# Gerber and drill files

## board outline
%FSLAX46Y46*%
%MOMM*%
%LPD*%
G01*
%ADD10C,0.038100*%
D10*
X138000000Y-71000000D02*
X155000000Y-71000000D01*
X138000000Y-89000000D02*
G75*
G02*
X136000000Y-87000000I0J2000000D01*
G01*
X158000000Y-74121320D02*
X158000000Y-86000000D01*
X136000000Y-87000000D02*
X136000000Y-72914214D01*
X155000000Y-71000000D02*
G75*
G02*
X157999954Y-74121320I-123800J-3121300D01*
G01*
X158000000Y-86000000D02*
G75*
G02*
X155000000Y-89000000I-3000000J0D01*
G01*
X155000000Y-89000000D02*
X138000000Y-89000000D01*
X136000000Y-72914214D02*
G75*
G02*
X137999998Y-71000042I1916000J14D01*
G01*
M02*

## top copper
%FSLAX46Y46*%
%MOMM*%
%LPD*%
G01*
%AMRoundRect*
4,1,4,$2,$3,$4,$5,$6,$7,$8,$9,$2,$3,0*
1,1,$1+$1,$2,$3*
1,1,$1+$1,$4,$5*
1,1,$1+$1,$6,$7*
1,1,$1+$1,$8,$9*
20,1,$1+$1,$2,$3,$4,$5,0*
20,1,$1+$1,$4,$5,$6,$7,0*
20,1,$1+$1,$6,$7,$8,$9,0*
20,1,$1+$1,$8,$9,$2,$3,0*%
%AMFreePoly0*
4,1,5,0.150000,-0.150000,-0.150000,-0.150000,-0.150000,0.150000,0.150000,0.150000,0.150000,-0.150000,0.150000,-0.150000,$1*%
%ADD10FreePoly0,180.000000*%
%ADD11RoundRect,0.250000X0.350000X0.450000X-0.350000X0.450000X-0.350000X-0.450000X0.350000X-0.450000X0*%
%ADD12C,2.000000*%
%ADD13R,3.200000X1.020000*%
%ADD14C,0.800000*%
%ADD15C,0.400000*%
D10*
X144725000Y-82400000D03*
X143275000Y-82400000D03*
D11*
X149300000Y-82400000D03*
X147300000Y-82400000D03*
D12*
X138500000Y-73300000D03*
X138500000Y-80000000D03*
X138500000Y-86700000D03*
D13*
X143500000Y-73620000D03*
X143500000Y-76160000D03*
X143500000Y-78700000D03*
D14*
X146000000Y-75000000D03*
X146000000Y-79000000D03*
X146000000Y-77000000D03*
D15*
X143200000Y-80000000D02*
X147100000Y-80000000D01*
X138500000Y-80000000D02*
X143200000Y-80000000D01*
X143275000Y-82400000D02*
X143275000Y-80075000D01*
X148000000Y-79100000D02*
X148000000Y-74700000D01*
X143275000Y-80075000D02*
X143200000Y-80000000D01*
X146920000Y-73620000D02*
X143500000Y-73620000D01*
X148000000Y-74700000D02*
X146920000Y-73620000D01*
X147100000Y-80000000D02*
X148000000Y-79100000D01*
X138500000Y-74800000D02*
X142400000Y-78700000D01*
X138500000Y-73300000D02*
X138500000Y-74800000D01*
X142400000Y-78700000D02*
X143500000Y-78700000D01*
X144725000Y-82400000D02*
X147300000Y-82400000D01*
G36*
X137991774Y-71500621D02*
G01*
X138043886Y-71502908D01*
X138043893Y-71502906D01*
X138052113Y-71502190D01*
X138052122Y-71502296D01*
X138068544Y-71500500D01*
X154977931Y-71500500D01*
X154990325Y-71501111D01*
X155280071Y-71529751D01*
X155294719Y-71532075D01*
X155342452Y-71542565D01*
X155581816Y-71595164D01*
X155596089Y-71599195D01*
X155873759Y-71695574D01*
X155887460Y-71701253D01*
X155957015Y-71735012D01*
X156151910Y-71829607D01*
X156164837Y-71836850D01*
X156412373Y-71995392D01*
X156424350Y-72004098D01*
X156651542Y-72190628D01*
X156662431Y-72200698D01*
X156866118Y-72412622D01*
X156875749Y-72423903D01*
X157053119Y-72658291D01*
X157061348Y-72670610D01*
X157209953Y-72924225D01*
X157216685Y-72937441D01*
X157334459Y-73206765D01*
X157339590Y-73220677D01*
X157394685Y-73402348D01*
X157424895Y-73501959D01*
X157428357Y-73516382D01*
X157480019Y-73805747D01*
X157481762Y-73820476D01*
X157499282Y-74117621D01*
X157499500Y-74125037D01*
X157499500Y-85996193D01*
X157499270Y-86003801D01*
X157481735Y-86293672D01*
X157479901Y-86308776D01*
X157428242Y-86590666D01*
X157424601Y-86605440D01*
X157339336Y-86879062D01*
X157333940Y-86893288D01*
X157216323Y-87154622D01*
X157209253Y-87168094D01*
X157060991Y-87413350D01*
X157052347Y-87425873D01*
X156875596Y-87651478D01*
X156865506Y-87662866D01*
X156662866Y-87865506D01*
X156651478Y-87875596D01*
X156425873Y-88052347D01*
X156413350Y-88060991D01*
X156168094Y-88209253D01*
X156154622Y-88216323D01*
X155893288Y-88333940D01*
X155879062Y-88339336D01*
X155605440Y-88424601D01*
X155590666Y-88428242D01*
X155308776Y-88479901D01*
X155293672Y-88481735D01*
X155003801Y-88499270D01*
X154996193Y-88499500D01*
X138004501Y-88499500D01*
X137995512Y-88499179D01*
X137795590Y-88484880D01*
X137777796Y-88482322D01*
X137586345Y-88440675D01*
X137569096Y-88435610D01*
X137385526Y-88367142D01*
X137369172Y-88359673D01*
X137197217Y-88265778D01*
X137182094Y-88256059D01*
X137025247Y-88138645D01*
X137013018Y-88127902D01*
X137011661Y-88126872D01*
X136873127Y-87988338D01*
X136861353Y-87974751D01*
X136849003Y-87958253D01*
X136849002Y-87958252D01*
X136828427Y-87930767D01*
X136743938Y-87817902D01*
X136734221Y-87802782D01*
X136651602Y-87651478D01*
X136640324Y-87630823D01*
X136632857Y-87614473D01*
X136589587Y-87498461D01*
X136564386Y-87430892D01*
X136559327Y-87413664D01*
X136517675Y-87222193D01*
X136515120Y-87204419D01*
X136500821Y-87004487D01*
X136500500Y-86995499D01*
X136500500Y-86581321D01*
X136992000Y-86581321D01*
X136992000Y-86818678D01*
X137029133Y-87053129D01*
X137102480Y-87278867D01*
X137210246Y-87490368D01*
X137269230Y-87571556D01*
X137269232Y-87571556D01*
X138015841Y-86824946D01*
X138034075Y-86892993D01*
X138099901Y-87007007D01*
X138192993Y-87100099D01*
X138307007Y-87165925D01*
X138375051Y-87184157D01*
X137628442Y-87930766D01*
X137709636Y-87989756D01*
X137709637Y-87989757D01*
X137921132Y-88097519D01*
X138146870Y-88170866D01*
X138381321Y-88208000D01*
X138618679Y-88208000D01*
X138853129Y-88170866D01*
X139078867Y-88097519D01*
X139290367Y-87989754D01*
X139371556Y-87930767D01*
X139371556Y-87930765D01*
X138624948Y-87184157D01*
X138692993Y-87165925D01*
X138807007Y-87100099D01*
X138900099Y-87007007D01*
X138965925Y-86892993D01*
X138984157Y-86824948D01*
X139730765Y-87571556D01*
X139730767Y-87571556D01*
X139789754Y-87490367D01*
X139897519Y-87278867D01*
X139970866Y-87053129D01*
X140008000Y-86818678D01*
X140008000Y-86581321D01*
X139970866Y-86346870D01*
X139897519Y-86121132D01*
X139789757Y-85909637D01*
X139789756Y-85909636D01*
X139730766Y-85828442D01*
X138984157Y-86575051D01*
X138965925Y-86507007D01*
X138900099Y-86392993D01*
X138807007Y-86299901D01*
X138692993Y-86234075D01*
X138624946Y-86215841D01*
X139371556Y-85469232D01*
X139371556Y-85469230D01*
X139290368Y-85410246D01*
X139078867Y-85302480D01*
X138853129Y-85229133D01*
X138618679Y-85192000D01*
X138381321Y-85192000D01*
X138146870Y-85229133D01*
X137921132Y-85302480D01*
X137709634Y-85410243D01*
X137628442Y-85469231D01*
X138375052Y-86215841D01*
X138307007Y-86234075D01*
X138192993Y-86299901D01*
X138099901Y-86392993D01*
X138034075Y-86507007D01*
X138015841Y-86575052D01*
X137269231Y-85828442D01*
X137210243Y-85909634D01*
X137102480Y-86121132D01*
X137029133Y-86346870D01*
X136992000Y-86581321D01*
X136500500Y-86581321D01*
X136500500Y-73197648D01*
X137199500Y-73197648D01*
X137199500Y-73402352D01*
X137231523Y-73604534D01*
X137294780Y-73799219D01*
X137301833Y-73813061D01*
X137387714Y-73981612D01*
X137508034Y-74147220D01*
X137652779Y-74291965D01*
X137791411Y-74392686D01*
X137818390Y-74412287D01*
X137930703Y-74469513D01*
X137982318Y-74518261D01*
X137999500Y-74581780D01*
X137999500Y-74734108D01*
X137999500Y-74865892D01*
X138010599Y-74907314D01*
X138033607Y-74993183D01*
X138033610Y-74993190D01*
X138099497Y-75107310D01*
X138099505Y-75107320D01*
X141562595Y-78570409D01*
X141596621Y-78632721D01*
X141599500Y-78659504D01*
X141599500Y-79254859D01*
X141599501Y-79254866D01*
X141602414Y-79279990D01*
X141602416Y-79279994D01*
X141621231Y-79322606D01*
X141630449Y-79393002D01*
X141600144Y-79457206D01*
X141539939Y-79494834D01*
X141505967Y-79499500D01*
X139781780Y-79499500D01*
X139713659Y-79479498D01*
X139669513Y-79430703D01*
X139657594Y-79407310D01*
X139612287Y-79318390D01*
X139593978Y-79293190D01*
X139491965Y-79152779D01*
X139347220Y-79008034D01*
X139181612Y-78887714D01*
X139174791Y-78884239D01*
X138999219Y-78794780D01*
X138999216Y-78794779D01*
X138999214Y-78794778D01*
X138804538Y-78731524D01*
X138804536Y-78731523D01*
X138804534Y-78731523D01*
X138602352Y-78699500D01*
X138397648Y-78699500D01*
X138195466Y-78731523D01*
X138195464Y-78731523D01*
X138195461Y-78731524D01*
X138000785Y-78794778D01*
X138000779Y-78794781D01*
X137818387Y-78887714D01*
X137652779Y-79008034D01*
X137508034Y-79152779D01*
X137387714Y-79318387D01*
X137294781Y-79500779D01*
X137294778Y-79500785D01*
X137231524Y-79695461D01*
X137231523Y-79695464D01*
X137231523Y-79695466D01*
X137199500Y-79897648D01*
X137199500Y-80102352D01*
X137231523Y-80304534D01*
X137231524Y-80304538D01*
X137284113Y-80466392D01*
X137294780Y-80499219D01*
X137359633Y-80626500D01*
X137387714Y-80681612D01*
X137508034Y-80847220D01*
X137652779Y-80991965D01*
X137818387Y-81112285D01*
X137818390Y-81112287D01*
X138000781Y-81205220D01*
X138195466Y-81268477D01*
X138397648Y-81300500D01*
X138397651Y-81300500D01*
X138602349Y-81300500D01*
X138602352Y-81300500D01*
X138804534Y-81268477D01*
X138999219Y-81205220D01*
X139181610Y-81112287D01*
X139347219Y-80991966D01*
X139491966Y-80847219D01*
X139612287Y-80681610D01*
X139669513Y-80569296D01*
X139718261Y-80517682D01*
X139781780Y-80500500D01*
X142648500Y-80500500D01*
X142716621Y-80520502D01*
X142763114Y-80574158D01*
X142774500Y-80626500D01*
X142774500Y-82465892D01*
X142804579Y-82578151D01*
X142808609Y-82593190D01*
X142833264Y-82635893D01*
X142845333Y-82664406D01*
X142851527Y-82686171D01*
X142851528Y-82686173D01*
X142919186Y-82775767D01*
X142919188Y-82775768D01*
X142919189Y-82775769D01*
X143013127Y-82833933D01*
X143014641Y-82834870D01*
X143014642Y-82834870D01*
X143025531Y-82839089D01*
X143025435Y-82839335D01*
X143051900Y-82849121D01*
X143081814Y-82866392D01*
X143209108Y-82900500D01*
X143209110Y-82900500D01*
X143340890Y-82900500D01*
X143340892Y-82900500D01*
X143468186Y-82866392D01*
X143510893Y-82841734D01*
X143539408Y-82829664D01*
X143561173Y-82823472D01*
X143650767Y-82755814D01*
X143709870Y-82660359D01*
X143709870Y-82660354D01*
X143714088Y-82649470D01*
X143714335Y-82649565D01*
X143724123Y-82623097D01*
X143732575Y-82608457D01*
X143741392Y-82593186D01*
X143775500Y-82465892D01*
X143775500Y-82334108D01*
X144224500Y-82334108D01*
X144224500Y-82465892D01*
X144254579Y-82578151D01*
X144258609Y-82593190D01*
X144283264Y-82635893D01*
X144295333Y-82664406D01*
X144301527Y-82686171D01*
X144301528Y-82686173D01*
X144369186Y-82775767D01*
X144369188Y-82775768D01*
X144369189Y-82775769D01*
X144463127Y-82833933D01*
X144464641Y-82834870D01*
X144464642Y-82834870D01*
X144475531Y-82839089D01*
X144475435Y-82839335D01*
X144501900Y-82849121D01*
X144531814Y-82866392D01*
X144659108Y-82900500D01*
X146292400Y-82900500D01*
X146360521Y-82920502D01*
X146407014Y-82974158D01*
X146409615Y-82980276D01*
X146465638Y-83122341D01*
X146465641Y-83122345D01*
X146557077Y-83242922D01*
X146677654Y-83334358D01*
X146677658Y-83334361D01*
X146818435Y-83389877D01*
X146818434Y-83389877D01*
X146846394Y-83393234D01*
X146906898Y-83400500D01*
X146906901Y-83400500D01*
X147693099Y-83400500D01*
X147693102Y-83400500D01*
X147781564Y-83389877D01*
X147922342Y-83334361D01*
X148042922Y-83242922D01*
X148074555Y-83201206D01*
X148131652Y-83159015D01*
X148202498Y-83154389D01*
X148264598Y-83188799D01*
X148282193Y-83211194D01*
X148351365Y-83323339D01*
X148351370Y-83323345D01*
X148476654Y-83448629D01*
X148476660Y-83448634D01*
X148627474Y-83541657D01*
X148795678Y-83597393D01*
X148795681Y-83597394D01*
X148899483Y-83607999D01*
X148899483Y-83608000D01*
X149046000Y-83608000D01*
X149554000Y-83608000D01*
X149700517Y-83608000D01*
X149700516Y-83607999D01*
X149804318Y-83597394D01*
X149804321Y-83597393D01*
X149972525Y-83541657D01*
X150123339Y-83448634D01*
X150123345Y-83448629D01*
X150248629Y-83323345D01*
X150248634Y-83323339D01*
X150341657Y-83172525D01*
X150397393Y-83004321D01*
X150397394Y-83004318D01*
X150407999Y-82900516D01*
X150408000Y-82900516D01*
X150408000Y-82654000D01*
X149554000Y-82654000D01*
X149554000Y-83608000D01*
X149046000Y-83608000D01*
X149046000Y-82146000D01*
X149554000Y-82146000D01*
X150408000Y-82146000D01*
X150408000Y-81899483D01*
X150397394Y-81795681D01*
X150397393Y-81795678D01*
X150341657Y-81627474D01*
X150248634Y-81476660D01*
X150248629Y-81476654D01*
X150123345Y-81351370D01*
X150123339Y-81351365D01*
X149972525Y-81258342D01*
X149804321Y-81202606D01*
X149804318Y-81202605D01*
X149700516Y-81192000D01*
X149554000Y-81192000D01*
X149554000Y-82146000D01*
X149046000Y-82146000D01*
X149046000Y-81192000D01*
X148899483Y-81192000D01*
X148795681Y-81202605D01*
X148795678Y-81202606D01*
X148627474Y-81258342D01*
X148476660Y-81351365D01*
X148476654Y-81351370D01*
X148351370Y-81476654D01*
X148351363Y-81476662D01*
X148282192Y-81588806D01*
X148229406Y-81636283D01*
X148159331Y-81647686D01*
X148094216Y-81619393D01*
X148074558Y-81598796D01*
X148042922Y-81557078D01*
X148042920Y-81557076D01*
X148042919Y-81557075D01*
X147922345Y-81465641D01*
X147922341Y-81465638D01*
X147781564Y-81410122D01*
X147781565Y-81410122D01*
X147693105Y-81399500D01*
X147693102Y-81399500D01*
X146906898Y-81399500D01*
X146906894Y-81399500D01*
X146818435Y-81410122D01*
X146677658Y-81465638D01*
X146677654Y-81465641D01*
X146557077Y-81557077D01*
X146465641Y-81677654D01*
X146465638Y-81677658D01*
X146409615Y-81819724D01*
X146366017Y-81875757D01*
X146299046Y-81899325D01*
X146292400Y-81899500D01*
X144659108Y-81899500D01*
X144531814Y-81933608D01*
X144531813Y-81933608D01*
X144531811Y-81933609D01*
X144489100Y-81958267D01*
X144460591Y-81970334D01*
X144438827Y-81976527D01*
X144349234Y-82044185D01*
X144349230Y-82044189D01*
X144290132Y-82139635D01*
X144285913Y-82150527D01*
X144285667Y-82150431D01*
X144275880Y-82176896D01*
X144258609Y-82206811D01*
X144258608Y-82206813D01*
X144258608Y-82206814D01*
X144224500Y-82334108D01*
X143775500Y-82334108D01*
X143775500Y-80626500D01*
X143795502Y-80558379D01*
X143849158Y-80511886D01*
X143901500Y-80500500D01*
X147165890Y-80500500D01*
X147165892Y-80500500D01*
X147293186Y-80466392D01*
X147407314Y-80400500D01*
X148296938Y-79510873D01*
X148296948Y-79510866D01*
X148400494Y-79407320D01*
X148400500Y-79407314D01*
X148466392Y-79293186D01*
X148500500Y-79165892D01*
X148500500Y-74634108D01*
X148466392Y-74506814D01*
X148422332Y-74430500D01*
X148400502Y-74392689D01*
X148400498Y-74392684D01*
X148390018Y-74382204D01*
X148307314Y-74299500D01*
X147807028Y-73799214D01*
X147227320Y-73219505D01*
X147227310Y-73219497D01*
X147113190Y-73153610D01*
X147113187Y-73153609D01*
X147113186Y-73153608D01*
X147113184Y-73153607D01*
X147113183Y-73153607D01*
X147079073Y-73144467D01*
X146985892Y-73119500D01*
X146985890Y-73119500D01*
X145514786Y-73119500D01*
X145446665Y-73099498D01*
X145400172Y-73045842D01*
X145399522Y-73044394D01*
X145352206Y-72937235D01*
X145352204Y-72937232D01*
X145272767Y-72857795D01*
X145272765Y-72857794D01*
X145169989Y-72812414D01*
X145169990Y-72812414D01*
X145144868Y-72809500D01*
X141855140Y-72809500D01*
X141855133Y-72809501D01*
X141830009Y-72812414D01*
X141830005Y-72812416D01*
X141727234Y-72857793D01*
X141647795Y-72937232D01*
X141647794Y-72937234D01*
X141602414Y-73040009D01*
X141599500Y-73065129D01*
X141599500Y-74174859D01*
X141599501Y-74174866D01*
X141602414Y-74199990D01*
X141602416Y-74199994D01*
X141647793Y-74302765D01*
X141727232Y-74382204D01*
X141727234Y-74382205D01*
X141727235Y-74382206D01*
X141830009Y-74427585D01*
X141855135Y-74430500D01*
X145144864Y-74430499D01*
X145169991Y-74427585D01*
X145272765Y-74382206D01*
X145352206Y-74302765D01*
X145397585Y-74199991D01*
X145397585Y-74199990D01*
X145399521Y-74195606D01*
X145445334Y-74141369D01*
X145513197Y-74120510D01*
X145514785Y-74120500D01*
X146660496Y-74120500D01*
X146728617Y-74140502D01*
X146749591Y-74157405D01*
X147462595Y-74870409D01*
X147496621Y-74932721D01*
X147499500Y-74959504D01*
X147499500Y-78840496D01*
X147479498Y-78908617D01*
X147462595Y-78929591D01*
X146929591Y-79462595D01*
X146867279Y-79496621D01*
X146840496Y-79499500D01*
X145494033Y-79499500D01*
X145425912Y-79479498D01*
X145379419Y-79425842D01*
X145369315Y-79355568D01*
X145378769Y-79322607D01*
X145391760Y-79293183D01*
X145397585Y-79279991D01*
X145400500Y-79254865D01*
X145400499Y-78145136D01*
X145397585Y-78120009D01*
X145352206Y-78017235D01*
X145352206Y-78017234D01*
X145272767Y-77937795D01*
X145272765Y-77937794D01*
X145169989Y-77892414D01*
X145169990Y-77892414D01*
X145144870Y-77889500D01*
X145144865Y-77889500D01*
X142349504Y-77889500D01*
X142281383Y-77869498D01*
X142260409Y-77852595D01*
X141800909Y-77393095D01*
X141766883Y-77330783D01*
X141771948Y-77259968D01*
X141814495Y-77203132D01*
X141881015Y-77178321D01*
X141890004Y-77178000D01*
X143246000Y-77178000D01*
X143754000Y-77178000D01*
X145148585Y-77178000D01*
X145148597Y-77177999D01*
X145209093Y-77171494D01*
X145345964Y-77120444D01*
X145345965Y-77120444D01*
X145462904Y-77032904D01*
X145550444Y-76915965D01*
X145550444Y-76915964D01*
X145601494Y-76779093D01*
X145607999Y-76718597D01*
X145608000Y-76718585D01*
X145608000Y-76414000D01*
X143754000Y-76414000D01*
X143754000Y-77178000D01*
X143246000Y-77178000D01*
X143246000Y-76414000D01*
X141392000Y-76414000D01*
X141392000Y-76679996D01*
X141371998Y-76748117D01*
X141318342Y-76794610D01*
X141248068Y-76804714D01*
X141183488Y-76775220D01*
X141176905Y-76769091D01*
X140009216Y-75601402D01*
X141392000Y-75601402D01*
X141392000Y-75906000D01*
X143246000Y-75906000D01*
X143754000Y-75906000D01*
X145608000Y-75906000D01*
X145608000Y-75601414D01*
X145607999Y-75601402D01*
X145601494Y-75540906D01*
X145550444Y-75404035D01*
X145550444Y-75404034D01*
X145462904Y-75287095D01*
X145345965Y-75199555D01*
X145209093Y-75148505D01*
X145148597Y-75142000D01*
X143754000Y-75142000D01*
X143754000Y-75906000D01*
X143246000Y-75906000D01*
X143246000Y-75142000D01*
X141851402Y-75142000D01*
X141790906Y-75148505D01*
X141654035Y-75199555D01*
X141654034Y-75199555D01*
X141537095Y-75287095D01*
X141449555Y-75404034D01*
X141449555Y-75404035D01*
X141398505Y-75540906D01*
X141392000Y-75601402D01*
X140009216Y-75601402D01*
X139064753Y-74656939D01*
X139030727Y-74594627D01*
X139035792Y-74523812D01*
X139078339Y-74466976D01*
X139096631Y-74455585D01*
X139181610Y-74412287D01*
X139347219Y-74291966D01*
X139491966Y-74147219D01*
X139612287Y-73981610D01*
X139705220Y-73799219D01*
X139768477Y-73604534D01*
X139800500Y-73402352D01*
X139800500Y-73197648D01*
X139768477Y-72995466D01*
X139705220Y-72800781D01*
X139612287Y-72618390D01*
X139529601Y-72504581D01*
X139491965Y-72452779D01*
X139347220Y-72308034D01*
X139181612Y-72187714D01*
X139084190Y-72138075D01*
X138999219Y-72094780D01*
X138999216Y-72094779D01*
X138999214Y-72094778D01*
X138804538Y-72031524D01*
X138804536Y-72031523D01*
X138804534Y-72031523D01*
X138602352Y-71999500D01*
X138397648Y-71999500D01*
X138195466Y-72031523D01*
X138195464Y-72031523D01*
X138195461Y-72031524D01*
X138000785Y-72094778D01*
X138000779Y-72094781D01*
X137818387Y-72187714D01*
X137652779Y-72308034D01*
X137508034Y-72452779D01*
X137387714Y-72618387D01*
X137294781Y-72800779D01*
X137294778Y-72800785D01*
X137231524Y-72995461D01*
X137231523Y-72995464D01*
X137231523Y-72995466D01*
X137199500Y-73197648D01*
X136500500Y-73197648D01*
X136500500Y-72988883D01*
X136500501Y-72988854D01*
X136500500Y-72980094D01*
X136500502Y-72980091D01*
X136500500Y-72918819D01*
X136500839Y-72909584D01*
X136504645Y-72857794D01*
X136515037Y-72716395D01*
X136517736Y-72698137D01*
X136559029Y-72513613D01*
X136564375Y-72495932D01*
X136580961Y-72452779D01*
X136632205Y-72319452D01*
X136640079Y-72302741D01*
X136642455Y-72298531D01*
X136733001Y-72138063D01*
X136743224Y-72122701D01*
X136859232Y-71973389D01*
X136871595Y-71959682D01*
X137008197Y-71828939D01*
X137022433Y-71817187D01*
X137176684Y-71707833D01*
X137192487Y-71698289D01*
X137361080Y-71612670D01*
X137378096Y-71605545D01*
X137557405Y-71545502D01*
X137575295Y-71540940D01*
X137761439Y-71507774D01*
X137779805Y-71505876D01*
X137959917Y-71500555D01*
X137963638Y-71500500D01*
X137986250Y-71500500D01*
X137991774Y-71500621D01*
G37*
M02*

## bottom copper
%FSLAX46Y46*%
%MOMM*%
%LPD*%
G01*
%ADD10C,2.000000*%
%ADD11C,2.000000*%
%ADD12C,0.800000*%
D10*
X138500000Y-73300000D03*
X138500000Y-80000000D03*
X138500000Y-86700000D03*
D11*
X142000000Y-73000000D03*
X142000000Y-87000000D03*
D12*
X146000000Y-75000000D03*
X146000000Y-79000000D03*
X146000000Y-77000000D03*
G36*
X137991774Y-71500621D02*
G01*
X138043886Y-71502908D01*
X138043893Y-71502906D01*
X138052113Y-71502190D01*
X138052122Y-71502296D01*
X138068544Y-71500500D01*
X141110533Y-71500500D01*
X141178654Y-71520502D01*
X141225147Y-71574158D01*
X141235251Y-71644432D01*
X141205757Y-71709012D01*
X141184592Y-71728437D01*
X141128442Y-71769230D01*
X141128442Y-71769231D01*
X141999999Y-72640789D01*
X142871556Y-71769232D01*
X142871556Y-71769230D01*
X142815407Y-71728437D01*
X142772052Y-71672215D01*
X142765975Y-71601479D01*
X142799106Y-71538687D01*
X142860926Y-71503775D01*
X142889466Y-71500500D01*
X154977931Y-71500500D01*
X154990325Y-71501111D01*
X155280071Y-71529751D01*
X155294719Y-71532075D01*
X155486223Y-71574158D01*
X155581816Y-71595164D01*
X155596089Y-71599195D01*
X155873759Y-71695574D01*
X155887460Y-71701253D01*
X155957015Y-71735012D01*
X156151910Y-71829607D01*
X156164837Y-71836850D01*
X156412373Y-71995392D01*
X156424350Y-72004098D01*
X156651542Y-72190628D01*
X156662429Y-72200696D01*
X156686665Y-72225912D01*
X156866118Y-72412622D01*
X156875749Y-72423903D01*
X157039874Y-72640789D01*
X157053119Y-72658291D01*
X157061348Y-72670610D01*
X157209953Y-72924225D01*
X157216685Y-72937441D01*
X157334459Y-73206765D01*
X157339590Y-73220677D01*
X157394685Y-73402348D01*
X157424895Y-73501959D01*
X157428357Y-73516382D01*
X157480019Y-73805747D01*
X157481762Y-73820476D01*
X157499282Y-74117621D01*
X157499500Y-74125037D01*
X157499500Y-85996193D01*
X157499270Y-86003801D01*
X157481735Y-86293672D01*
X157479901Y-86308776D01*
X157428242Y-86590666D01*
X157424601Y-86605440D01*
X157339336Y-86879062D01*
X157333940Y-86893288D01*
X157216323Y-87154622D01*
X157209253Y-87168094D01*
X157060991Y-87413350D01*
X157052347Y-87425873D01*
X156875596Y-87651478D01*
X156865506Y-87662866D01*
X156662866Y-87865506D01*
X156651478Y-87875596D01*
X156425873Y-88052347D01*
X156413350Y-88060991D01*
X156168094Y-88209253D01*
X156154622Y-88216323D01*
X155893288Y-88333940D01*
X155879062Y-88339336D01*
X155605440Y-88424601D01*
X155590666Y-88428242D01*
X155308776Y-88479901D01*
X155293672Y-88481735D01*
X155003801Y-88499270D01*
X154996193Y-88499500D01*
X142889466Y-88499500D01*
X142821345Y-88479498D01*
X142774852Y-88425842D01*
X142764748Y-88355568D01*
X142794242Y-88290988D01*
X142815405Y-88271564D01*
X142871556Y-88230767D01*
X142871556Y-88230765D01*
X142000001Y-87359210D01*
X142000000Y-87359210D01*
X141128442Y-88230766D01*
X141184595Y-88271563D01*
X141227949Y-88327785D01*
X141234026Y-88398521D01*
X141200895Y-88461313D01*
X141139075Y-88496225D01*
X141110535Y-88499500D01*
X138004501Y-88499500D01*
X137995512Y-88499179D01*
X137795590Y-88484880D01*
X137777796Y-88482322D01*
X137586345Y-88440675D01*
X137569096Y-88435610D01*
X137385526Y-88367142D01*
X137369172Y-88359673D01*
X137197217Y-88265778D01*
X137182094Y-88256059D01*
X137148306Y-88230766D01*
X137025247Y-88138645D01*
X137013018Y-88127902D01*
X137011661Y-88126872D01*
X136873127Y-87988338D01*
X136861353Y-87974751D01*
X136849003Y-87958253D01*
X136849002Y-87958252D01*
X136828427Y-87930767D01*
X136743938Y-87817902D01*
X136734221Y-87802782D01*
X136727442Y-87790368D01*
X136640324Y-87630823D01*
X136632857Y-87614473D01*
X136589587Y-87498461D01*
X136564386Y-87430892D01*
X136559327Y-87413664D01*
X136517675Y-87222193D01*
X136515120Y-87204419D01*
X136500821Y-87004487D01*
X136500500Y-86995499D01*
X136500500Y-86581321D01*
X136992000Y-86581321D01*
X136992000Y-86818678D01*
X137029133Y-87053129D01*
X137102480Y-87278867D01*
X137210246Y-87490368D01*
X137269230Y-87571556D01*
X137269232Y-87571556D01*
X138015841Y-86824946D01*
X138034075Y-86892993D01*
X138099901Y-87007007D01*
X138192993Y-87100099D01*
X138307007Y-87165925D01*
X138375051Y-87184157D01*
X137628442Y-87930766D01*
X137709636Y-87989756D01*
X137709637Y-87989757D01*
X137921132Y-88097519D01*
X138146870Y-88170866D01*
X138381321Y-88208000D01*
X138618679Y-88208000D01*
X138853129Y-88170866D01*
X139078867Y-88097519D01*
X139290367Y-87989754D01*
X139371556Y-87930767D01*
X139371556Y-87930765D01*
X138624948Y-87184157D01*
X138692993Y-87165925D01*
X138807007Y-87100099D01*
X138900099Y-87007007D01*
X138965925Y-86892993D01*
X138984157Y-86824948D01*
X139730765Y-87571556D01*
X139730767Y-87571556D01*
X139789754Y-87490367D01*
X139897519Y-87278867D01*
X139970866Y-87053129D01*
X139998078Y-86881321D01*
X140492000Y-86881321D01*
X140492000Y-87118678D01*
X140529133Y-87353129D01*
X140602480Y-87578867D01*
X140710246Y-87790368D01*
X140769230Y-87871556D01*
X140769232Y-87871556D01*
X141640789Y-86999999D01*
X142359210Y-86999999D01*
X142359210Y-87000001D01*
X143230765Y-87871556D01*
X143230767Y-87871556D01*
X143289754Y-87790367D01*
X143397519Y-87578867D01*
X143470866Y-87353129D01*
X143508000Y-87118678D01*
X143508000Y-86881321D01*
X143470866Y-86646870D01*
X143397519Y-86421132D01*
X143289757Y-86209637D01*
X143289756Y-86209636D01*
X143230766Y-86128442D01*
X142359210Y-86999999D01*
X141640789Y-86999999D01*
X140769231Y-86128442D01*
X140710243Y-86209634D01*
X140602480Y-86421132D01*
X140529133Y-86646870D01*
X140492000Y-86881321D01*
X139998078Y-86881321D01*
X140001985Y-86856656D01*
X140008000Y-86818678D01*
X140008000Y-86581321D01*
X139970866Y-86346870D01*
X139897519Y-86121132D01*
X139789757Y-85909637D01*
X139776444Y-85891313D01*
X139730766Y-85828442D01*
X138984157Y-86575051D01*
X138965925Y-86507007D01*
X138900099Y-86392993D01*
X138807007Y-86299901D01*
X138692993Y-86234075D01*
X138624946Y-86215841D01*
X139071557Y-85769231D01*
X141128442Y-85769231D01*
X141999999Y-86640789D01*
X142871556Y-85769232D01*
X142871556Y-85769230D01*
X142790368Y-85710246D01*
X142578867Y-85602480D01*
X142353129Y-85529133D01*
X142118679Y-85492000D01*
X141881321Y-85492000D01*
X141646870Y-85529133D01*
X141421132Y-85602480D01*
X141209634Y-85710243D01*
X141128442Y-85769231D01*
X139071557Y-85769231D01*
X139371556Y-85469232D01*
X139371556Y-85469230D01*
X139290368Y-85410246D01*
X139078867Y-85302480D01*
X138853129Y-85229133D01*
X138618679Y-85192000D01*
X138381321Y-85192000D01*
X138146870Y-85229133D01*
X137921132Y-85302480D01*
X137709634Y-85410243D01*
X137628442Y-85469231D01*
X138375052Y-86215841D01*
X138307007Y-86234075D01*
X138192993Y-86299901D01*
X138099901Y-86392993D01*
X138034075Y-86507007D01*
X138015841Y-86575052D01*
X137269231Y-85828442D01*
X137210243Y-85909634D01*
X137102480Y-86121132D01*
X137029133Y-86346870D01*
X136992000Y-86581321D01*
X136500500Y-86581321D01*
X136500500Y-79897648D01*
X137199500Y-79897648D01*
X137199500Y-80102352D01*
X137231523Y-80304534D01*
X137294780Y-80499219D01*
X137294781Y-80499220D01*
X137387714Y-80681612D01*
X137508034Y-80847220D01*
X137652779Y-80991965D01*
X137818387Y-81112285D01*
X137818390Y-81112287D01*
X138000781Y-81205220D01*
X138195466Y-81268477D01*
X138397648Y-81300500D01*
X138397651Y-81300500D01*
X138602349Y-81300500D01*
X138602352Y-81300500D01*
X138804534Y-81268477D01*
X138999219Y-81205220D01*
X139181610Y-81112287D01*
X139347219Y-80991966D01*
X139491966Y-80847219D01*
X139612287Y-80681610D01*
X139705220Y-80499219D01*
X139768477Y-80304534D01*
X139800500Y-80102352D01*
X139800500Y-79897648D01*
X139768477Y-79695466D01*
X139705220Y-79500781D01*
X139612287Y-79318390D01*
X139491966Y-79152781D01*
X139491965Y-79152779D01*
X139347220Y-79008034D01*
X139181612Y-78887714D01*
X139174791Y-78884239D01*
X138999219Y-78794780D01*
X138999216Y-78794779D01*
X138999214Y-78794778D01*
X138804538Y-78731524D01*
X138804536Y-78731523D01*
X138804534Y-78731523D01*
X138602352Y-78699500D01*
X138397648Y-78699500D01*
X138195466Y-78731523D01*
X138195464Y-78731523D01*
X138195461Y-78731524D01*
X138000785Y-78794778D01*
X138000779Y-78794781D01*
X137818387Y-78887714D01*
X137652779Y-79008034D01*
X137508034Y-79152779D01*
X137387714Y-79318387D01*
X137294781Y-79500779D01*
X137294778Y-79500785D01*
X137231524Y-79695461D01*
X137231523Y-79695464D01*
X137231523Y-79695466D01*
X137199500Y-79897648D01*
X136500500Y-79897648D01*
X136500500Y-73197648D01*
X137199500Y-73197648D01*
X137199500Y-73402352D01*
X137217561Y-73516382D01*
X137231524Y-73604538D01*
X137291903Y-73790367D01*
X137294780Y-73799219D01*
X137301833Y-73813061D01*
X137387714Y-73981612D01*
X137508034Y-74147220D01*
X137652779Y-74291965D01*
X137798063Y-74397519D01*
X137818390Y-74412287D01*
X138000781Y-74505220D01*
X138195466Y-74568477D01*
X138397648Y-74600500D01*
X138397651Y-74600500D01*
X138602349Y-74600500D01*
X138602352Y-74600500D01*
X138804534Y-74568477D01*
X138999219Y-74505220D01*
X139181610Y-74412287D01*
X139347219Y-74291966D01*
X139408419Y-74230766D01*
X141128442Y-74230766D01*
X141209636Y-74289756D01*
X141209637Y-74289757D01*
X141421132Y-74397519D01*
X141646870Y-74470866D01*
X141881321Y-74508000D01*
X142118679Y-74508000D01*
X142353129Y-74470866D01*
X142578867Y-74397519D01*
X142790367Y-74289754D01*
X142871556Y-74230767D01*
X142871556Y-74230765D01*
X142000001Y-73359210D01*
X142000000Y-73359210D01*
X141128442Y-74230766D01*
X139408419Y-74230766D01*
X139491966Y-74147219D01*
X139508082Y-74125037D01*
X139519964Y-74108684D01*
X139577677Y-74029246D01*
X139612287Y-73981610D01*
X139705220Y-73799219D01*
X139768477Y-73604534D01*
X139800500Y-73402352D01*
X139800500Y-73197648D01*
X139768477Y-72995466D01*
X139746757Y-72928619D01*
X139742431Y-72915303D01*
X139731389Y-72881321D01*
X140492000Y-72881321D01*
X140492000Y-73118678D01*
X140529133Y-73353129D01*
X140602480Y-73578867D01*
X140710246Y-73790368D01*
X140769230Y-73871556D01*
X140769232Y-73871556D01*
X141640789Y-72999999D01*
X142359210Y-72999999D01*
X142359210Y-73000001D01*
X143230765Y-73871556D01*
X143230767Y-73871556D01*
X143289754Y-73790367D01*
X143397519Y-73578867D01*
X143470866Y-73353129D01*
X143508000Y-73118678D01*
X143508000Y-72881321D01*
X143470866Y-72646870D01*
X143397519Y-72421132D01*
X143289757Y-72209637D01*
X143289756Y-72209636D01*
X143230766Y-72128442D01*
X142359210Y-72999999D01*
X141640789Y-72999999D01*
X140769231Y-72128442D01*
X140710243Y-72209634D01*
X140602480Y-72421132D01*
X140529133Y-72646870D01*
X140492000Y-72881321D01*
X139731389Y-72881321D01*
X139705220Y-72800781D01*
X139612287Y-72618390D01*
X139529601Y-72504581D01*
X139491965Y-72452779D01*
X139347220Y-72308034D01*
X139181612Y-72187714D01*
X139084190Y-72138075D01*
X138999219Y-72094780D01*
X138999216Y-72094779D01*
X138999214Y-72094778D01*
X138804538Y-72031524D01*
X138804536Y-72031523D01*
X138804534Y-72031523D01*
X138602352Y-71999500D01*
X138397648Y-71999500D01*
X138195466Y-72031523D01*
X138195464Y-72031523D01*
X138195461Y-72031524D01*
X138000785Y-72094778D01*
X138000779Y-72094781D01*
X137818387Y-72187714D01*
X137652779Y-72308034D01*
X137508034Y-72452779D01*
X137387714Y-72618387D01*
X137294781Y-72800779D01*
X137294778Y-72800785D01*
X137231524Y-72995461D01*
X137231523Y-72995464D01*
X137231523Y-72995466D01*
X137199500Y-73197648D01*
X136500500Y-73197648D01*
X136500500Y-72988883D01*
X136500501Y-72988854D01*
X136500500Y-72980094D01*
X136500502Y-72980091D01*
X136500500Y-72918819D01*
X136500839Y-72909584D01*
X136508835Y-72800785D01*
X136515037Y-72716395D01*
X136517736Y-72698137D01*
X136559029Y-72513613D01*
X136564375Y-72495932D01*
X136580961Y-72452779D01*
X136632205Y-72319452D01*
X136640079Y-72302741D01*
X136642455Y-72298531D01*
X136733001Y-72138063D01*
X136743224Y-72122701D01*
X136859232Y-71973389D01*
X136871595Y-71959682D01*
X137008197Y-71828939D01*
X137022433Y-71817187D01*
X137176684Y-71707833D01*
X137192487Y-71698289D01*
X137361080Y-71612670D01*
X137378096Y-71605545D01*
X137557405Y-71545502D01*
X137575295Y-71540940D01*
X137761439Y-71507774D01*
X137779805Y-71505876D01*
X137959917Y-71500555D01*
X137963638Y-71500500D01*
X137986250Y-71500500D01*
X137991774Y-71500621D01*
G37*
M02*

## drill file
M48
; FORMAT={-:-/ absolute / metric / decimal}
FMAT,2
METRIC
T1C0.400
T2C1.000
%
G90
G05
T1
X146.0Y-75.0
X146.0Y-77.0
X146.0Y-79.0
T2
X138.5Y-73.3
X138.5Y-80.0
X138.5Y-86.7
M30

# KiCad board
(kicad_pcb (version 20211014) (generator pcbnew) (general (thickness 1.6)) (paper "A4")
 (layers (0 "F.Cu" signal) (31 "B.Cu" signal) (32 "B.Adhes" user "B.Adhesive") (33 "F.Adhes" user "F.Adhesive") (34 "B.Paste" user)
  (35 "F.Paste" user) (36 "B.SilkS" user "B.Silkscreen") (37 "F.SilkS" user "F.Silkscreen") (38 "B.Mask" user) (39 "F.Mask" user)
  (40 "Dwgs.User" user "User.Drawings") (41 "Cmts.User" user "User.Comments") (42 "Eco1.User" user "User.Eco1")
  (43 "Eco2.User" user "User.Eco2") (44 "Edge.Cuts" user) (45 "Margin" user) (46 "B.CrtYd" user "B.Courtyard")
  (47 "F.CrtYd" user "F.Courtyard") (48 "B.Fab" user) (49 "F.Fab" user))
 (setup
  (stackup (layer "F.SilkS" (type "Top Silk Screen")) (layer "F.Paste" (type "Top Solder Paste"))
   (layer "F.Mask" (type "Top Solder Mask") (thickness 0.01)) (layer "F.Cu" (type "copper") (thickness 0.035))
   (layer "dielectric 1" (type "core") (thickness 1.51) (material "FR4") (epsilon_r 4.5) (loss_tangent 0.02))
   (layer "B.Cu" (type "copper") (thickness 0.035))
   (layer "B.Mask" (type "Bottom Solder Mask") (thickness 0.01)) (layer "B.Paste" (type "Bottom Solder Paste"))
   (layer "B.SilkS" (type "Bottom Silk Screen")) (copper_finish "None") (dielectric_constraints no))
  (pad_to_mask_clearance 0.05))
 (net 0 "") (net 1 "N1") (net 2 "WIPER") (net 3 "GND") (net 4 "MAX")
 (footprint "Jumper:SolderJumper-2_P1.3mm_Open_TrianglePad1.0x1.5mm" (layer "F.Cu") (at 144 82.4 180)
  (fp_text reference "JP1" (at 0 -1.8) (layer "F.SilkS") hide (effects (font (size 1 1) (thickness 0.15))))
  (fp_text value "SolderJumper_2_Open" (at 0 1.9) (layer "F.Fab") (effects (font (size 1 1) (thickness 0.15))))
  (pad "1" smd custom (at -0.725 0 180) (size 0.3 0.3) (layers "F.Cu" "F.Mask") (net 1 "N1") (zone_connect 2)
   (options (clearance outline) (anchor rect)) (primitives))
  (pad "2" smd custom (at 0.725 0 180) (size 0.3 0.3) (layers "F.Cu" "F.Mask") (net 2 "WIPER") (zone_connect 2)
   (options (clearance outline) (anchor rect)) (primitives)))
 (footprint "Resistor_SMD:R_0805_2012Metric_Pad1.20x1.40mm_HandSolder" (layer "F.Cu") (at 148.3 82.4 180)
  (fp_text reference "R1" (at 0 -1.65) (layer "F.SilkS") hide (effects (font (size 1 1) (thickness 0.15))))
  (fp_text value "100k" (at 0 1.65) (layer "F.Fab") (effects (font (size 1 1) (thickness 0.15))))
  (pad "1" smd roundrect (at -1 0 180) (size 1.2 1.4) (layers "F.Cu" "F.Paste" "F.Mask") (roundrect_rratio 0.208333) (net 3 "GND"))
  (pad "2" smd roundrect (at 1 0 180) (size 1.2 1.4) (layers "F.Cu" "F.Paste" "F.Mask") (roundrect_rratio 0.208333) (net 1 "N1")))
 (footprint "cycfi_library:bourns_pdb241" (layer "F.Cu") (at 138.5 80)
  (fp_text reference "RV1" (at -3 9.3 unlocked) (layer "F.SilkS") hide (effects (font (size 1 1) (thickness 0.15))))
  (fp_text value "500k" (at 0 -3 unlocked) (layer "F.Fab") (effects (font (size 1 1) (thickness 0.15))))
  (pad "1" thru_hole circle (at 0 -6.7) (size 2 2) (drill 1) (layers *.Cu *.Mask) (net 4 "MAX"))
  (pad "2" thru_hole circle (at 0 0) (size 2 2) (drill 1) (layers *.Cu *.Mask) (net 2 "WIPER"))
  (pad "3" thru_hole circle (at 0 6.7) (size 2 2) (drill 1) (layers *.Cu *.Mask) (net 3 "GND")))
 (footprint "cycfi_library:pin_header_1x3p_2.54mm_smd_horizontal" (layer "F.Cu") (at 143.5 73.62)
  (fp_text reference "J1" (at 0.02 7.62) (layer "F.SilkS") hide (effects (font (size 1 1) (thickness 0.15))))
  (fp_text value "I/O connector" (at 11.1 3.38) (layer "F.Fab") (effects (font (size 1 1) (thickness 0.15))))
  (pad "1" smd rect (at 0 0) (size 3.2 1.02) (layers "F.Cu" "F.Paste" "F.Mask") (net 2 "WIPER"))
  (pad "2" smd rect (at 0 2.54) (size 3.2 1.02) (layers "F.Cu" "F.Paste" "F.Mask") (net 3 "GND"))
  (pad "3" smd rect (at 0 5.08) (size 3.2 1.02) (layers "F.Cu" "F.Paste" "F.Mask") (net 4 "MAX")))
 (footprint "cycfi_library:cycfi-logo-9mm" (layer "F.Cu") (at 150.7 85.7)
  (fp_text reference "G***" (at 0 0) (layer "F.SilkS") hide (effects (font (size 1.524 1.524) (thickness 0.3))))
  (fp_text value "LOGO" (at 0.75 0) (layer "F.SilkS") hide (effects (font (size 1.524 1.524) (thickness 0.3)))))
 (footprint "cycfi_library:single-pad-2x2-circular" (layer "B.Cu") (at 142 73 180)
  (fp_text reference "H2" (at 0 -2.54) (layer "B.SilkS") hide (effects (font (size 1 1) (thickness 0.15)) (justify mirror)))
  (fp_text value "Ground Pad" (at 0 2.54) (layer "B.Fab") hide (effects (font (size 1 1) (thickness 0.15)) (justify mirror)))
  (pad "1" smd circle (at 0 0 180) (size 2 2) (layers "B.Cu" "B.Paste" "B.Mask") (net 3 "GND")))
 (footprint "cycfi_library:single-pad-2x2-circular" (layer "B.Cu") (at 142 87 180)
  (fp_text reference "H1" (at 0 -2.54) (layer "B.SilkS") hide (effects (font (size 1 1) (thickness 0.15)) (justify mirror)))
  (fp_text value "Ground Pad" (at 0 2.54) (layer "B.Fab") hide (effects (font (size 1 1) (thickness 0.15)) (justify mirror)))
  (pad "1" smd circle (at 0 0 180) (size 2 2) (layers "B.Cu" "B.Paste" "B.Mask") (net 3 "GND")))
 (gr_line (start 138 71) (end 155 71) (layer "Edge.Cuts") (width 0.0381))
 (gr_arc (start 138 89) (mid 136.585786 88.414214) (end 136 87) (layer "Edge.Cuts") (width 0.0381))
 (gr_line (start 158 74.12132) (end 158 86) (layer "Edge.Cuts") (width 0.0381))
 (gr_line (start 136 87) (end 136 72.914214) (layer "Edge.Cuts") (width 0.0381))
 (gr_arc (start 155 71) (mid 157.128402 71.956683) (end 158 74.12132) (layer "Edge.Cuts") (width 0.0381))
 (gr_arc (start 158 86) (mid 157.121318 88.121318) (end 155 89) (layer "Edge.Cuts") (width 0.0381))
 (gr_line (start 155 89) (end 138 89) (layer "Edge.Cuts") (width 0.0381))
 (gr_arc (start 136 72.914214) (mid 136.591204 71.529971) (end 138 71) (layer "Edge.Cuts") (width 0.0381))
 (segment (start 143.2 80) (end 147.1 80) (width 0.4) (layer "F.Cu") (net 2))
 (segment (start 138.5 80) (end 143.2 80) (width 0.4) (layer "F.Cu") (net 2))
 (segment (start 143.275 82.4) (end 143.275 80.075) (width 0.4) (layer "F.Cu") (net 2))
 (segment (start 148 79.1) (end 148 74.7) (width 0.4) (layer "F.Cu") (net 2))
 (segment (start 143.275 80.075) (end 143.2 80) (width 0.4) (layer "F.Cu") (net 2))
 (segment (start 146.92 73.62) (end 143.5 73.62) (width 0.4) (layer "F.Cu") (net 2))
 (segment (start 148 74.7) (end 146.92 73.62) (width 0.4) (layer "F.Cu") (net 2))
 (segment (start 147.1 80) (end 148 79.1) (width 0.4) (layer "F.Cu") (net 2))
 (via (at 146 75) (size 0.8) (drill 0.4) (layers "F.Cu" "B.Cu") (free) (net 3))
 (via (at 146 79) (size 0.8) (drill 0.4) (layers "F.Cu" "B.Cu") (free) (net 3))
 (via (at 146 77) (size 0.8) (drill 0.4) (layers "F.Cu" "B.Cu") (free) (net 3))
 (segment (start 138.5 74.8) (end 142.4 78.7) (width 0.4) (layer "F.Cu") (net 4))
 (segment (start 138.5 73.3) (end 138.5 74.8) (width 0.4) (layer "F.Cu") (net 4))
 (segment (start 142.4 78.7) (end 143.5 78.7) (width 0.4) (layer "F.Cu") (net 4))
 (segment (start 144.725 82.4) (end 147.3 82.4) (width 0.4) (layer "F.Cu") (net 1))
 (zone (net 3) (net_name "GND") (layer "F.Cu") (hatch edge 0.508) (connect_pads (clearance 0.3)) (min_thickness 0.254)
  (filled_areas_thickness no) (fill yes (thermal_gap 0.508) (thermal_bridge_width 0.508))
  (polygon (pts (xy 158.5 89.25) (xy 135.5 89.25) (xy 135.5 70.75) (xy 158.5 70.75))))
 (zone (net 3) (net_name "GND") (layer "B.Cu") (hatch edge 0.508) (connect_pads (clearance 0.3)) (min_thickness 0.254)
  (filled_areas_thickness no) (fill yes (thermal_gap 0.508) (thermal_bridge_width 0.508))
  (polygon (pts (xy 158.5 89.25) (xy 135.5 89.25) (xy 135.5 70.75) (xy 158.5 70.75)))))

